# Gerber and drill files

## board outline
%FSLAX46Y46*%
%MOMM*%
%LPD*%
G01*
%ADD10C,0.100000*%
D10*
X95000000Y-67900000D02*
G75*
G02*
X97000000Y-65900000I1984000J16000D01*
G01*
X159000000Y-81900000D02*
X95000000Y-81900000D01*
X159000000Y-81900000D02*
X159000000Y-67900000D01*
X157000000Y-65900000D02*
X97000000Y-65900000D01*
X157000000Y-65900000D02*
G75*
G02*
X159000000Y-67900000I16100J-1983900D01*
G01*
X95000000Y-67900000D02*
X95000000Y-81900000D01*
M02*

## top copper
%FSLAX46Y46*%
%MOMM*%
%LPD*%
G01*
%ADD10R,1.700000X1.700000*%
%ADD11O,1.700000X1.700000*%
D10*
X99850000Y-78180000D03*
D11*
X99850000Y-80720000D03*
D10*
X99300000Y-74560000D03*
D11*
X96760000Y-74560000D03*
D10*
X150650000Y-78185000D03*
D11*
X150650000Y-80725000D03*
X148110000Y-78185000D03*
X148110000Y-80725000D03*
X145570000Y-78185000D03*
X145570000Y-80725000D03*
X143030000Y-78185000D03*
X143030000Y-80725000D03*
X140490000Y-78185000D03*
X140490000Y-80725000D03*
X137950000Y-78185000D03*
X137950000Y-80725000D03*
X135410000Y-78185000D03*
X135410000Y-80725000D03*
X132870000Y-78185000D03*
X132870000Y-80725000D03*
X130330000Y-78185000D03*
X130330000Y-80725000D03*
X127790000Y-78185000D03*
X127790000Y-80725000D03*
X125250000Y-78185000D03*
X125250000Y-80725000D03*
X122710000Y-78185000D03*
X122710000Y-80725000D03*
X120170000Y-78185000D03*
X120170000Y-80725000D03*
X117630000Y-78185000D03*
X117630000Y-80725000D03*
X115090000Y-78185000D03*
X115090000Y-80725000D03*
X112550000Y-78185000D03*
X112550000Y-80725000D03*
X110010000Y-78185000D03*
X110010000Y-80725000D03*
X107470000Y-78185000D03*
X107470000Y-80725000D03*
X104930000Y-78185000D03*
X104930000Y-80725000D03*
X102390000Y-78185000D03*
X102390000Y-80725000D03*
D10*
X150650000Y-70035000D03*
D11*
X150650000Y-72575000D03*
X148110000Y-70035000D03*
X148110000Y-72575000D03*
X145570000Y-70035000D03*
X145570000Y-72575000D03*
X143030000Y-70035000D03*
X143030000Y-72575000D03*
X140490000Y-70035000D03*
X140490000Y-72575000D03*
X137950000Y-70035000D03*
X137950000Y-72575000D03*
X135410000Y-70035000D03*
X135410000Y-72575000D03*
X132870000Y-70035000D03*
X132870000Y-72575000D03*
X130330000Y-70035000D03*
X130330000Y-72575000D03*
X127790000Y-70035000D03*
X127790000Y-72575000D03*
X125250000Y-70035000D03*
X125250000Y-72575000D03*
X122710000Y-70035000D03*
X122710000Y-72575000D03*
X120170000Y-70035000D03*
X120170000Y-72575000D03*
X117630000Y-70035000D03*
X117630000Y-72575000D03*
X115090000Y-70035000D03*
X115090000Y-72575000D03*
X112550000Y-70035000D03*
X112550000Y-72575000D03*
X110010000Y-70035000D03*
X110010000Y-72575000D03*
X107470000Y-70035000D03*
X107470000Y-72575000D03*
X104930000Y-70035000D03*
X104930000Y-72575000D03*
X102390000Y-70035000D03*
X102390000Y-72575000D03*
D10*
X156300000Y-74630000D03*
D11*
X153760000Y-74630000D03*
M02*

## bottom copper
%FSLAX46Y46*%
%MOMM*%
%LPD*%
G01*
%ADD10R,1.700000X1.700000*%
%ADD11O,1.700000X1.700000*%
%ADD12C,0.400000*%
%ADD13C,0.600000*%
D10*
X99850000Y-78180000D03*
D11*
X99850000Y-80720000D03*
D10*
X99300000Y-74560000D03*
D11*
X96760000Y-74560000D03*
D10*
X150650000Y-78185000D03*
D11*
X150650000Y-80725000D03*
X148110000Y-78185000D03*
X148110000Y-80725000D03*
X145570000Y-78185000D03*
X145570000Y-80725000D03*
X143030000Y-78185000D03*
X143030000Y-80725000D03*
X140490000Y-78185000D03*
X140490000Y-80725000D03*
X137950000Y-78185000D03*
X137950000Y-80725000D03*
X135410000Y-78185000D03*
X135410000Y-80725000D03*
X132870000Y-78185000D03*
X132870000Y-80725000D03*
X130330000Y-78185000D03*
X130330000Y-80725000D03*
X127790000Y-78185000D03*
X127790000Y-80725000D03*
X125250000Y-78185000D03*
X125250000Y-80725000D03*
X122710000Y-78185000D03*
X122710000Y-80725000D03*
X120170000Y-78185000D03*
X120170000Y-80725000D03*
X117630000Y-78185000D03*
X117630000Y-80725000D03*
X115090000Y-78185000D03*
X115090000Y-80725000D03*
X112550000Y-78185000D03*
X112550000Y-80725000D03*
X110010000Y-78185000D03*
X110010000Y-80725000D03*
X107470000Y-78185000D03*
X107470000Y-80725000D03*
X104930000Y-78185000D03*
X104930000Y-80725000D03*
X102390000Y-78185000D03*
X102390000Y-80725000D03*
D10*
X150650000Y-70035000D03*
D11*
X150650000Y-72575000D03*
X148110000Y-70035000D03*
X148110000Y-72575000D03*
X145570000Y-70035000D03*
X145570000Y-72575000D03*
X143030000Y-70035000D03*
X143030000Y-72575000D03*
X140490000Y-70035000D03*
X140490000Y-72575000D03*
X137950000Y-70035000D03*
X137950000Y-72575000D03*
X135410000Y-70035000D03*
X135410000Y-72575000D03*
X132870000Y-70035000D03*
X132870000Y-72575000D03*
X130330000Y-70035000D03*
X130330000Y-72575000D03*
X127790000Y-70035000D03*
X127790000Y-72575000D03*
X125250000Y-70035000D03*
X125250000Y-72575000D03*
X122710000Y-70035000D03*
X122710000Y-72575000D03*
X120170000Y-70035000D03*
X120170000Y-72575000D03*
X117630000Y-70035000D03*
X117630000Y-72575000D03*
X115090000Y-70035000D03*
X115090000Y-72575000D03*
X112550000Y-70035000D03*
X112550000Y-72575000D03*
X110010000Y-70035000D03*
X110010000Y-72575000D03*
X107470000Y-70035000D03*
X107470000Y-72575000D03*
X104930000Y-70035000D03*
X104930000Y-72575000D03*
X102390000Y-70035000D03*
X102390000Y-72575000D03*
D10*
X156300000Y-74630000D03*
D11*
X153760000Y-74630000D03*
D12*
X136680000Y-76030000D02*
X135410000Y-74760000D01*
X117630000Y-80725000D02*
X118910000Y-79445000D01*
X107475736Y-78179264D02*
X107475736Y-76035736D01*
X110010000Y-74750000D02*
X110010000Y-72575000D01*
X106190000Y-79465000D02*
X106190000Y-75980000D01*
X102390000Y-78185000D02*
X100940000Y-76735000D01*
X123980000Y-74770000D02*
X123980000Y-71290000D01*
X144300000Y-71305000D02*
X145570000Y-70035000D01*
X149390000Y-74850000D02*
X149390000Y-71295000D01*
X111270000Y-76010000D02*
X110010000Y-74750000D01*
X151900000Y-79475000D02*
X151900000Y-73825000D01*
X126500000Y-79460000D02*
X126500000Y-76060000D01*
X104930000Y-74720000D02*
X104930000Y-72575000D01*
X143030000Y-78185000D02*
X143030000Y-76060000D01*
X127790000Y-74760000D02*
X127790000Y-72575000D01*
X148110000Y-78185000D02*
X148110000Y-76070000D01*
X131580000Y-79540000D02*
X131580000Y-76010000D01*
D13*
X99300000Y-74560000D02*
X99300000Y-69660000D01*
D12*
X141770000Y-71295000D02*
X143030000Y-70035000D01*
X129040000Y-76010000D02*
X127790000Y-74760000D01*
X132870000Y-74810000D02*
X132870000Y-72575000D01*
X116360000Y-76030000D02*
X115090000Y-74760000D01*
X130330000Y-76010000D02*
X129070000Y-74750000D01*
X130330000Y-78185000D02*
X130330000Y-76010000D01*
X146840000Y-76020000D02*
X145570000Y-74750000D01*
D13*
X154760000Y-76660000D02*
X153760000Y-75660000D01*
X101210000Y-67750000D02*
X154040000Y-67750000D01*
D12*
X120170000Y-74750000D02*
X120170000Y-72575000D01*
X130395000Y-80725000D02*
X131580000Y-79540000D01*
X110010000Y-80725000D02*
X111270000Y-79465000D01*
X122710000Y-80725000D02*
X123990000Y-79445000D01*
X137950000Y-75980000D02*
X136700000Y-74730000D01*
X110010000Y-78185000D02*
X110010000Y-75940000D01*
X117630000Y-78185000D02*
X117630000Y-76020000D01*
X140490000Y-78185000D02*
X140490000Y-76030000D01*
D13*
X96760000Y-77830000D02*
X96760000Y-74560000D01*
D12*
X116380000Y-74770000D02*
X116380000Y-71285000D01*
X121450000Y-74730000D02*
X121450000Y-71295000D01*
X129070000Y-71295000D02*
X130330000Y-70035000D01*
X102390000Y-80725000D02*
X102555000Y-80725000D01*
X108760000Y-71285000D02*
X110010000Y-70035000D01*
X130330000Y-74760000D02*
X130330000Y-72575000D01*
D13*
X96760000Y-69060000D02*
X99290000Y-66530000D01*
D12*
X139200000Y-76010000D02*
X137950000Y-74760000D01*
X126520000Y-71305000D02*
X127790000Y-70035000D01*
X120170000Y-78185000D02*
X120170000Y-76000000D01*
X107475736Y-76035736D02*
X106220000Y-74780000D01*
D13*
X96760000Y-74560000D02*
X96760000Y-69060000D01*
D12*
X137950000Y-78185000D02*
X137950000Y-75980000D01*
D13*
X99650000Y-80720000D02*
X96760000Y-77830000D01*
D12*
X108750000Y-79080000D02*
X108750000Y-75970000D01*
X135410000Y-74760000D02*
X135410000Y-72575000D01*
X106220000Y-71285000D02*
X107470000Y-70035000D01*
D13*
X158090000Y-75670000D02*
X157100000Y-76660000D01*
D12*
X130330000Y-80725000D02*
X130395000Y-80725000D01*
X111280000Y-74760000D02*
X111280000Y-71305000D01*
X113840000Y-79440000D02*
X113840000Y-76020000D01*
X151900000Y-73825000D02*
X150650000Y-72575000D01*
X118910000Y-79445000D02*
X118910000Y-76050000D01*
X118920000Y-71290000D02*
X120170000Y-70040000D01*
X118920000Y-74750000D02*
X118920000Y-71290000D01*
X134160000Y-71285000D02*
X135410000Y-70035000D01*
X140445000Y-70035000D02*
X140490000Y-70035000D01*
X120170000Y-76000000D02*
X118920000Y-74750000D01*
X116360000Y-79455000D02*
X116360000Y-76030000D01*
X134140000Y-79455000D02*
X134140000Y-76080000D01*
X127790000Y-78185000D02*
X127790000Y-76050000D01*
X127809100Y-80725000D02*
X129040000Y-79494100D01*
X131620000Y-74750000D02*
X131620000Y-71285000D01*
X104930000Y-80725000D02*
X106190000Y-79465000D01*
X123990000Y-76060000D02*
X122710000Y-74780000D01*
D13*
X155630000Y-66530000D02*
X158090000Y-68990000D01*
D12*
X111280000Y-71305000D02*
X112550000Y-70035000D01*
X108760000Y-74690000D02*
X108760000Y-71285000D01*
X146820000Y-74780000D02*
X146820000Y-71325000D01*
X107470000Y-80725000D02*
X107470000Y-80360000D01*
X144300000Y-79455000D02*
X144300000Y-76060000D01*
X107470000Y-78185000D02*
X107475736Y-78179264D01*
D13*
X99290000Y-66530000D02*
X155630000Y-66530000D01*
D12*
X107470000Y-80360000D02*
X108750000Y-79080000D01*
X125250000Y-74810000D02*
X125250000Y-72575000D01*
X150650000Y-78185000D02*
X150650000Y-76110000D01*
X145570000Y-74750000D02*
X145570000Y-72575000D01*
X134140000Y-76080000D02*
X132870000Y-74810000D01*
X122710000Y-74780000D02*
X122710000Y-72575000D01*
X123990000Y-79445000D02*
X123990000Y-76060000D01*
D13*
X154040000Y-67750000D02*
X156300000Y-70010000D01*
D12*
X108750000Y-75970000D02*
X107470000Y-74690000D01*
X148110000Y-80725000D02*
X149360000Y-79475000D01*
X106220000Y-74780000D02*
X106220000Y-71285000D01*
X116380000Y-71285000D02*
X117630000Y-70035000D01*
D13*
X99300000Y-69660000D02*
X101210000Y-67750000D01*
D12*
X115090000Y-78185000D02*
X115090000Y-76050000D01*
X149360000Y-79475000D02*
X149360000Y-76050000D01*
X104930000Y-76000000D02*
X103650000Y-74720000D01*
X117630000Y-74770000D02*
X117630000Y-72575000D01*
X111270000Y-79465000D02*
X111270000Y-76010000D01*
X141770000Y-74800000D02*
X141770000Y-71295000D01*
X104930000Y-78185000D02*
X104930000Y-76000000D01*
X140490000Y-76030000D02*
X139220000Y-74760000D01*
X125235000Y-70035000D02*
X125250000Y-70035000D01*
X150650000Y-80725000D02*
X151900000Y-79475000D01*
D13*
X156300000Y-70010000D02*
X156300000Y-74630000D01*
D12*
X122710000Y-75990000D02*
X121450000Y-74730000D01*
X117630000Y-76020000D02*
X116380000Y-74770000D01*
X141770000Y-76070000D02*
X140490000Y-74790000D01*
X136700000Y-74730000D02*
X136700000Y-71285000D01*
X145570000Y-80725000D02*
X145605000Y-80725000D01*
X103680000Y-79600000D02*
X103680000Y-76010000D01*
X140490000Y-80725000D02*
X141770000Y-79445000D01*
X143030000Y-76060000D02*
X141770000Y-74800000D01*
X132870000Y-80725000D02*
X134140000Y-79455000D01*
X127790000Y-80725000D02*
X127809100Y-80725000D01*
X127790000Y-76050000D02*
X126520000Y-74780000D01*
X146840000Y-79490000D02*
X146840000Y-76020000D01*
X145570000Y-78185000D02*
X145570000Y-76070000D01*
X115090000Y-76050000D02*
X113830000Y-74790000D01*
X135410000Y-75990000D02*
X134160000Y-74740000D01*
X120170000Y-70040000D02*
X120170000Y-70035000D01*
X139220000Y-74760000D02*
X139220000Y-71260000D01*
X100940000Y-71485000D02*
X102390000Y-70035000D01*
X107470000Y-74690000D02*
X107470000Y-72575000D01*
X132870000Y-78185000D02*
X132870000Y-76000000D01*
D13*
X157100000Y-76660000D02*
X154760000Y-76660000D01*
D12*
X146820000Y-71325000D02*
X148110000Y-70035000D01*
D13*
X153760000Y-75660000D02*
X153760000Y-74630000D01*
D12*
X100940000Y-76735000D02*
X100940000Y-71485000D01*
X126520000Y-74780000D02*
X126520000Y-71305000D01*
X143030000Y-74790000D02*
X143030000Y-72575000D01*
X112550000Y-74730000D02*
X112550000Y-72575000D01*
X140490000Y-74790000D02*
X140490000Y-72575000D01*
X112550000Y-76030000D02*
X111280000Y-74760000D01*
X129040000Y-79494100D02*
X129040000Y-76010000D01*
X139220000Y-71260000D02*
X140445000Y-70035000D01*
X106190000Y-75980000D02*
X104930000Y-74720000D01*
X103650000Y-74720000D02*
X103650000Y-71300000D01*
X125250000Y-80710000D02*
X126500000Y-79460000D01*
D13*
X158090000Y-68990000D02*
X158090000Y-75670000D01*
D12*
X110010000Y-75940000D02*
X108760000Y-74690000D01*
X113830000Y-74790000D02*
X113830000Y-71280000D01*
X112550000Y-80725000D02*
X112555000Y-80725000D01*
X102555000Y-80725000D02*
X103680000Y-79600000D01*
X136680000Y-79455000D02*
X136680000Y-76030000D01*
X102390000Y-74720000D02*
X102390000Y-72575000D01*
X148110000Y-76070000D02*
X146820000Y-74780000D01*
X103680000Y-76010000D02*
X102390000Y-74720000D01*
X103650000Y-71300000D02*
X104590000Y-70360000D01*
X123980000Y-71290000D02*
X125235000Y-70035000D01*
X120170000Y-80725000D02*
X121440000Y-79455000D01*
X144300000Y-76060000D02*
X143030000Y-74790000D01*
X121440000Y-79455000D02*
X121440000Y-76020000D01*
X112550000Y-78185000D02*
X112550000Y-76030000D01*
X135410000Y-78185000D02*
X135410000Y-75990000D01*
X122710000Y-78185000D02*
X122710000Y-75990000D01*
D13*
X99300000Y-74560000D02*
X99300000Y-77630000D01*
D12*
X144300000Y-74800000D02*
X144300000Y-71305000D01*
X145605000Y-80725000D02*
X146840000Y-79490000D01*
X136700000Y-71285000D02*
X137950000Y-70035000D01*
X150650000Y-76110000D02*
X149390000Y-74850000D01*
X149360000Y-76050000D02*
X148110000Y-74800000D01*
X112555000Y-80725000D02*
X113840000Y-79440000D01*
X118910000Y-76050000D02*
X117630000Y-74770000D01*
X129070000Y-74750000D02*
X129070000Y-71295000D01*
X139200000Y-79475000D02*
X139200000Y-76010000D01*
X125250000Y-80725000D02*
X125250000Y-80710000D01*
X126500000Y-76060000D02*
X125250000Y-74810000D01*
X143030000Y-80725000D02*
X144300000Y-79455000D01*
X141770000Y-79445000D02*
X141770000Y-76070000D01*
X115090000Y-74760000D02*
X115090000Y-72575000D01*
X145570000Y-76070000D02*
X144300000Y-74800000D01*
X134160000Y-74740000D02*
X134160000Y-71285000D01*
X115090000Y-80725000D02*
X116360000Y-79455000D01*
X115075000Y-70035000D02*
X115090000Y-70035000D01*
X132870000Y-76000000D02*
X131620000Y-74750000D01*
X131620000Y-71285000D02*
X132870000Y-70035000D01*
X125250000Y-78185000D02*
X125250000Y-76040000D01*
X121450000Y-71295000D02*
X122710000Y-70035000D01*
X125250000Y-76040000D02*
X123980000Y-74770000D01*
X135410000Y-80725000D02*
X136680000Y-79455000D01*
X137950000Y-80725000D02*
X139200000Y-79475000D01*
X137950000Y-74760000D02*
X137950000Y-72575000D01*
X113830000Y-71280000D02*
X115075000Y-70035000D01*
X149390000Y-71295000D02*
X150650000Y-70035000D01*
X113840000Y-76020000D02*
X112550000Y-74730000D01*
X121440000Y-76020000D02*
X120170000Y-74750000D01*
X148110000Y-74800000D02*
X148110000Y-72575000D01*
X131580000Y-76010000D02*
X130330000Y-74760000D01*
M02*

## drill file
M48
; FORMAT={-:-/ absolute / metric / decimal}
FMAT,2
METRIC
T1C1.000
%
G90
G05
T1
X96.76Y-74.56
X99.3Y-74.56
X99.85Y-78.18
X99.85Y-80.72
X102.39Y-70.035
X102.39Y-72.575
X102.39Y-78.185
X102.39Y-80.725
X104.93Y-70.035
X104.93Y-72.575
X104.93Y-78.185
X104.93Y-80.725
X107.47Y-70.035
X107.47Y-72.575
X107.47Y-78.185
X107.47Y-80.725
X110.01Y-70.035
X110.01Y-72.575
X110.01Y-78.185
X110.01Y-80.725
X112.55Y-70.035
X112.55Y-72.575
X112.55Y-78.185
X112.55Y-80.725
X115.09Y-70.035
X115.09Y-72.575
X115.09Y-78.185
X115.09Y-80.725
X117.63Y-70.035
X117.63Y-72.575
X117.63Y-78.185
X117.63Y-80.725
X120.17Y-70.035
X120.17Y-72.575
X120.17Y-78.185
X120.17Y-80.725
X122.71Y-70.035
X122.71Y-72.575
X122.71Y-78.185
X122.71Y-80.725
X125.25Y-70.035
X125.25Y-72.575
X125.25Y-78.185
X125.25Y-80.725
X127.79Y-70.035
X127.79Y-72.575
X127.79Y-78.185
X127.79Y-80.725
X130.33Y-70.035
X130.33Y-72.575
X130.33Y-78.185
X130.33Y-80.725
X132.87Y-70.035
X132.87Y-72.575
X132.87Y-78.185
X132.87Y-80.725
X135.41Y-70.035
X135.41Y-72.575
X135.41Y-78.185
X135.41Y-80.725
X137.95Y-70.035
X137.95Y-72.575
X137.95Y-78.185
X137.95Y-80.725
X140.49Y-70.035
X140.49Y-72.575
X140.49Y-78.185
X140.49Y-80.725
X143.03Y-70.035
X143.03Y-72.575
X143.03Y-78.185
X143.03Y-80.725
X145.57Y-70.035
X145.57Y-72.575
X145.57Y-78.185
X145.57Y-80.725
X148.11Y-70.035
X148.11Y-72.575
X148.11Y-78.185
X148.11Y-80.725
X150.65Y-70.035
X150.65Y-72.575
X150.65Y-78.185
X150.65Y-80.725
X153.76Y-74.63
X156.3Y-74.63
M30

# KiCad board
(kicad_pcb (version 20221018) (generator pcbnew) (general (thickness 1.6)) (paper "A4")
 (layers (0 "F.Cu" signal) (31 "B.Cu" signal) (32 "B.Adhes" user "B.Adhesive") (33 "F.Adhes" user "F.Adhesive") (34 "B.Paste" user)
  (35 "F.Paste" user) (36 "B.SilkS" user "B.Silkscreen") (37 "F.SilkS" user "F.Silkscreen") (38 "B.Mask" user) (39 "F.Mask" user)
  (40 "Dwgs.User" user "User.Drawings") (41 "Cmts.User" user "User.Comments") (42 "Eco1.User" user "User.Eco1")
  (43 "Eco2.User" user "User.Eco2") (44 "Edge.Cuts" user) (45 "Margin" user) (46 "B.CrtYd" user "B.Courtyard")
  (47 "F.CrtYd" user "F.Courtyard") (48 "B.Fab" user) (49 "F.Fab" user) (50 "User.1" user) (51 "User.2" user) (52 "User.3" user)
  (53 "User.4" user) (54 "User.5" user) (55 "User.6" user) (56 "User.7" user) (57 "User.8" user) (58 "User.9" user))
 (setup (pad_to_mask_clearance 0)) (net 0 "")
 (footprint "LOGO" (layer "F.Cu") (at 126.5 75.56)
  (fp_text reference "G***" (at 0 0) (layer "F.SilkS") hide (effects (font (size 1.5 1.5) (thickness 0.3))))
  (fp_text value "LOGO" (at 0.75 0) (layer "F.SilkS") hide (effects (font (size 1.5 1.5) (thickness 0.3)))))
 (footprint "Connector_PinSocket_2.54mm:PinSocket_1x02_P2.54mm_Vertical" (layer "B.Cu") (at 99.85 78.18 180)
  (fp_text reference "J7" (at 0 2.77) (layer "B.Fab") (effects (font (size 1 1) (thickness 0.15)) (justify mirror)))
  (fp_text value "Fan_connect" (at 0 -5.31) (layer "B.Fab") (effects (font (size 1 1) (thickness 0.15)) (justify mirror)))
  (pad "1" thru_hole rect (at 0 0 180) (size 1.7 1.7) (drill 1) (layers "*.Cu" "*.Mask"))
  (pad "2" thru_hole oval (at 0 -2.54 180) (size 1.7 1.7) (drill 1) (layers "*.Cu" "*.Mask")))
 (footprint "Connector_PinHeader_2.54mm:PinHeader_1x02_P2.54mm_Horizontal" (layer "B.Cu") (at 99.3 74.56 90)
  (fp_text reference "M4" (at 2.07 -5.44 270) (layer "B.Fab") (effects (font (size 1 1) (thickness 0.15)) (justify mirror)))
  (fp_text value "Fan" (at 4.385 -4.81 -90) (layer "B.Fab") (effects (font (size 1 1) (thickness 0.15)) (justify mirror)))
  (pad "1" thru_hole rect (at 0 0 90) (size 1.7 1.7) (drill 1) (layers "*.Cu" "*.Mask"))
  (pad "2" thru_hole oval (at 0 -2.54 90) (size 1.7 1.7) (drill 1) (layers "*.Cu" "*.Mask")))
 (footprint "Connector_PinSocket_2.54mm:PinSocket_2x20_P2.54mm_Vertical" (layer "B.Cu") (at 126.49 79.455 90)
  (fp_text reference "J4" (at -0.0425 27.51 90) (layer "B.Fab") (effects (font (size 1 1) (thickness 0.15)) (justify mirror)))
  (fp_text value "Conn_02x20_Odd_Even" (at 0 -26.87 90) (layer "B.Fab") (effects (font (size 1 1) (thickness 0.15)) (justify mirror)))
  (pad "1" thru_hole rect (at 1.27 24.16 90) (size 1.7 1.7) (drill 1) (layers "*.Cu" "*.Mask"))
  (pad "2" thru_hole oval (at -1.27 24.16 90) (size 1.7 1.7) (drill 1) (layers "*.Cu" "*.Mask"))
  (pad "3" thru_hole oval (at 1.27 21.62 90) (size 1.7 1.7) (drill 1) (layers "*.Cu" "*.Mask"))
  (pad "4" thru_hole oval (at -1.27 21.62 90) (size 1.7 1.7) (drill 1) (layers "*.Cu" "*.Mask"))
  (pad "5" thru_hole oval (at 1.27 19.08 90) (size 1.7 1.7) (drill 1) (layers "*.Cu" "*.Mask"))
  (pad "6" thru_hole oval (at -1.27 19.08 90) (size 1.7 1.7) (drill 1) (layers "*.Cu" "*.Mask"))
  (pad "7" thru_hole oval (at 1.27 16.54 90) (size 1.7 1.7) (drill 1) (layers "*.Cu" "*.Mask"))
  (pad "8" thru_hole oval (at -1.27 16.54 90) (size 1.7 1.7) (drill 1) (layers "*.Cu" "*.Mask"))
  (pad "9" thru_hole oval (at 1.27 14 90) (size 1.7 1.7) (drill 1) (layers "*.Cu" "*.Mask"))
  (pad "10" thru_hole oval (at -1.27 14 90) (size 1.7 1.7) (drill 1) (layers "*.Cu" "*.Mask"))
  (pad "11" thru_hole oval (at 1.27 11.46 90) (size 1.7 1.7) (drill 1) (layers "*.Cu" "*.Mask"))
  (pad "12" thru_hole oval (at -1.27 11.46 90) (size 1.7 1.7) (drill 1) (layers "*.Cu" "*.Mask"))
  (pad "13" thru_hole oval (at 1.27 8.92 90) (size 1.7 1.7) (drill 1) (layers "*.Cu" "*.Mask"))
  (pad "14" thru_hole oval (at -1.27 8.92 90) (size 1.7 1.7) (drill 1) (layers "*.Cu" "*.Mask"))
  (pad "15" thru_hole oval (at 1.27 6.38 90) (size 1.7 1.7) (drill 1) (layers "*.Cu" "*.Mask"))
  (pad "16" thru_hole oval (at -1.27 6.38 90) (size 1.7 1.7) (drill 1) (layers "*.Cu" "*.Mask"))
  (pad "17" thru_hole oval (at 1.27 3.84 90) (size 1.7 1.7) (drill 1) (layers "*.Cu" "*.Mask"))
  (pad "18" thru_hole oval (at -1.27 3.84 90) (size 1.7 1.7) (drill 1) (layers "*.Cu" "*.Mask"))
  (pad "19" thru_hole oval (at 1.27 1.3 90) (size 1.7 1.7) (drill 1) (layers "*.Cu" "*.Mask"))
  (pad "20" thru_hole oval (at -1.27 1.3 90) (size 1.7 1.7) (drill 1) (layers "*.Cu" "*.Mask"))
  (pad "21" thru_hole oval (at 1.27 -1.24 90) (size 1.7 1.7) (drill 1) (layers "*.Cu" "*.Mask"))
  (pad "22" thru_hole oval (at -1.27 -1.24 90) (size 1.7 1.7) (drill 1) (layers "*.Cu" "*.Mask"))
  (pad "23" thru_hole oval (at 1.27 -3.78 90) (size 1.7 1.7) (drill 1) (layers "*.Cu" "*.Mask"))
  (pad "24" thru_hole oval (at -1.27 -3.78 90) (size 1.7 1.7) (drill 1) (layers "*.Cu" "*.Mask"))
  (pad "25" thru_hole oval (at 1.27 -6.32 90) (size 1.7 1.7) (drill 1) (layers "*.Cu" "*.Mask"))
  (pad "26" thru_hole oval (at -1.27 -6.32 90) (size 1.7 1.7) (drill 1) (layers "*.Cu" "*.Mask"))
  (pad "27" thru_hole oval (at 1.27 -8.86 90) (size 1.7 1.7) (drill 1) (layers "*.Cu" "*.Mask"))
  (pad "28" thru_hole oval (at -1.27 -8.86 90) (size 1.7 1.7) (drill 1) (layers "*.Cu" "*.Mask"))
  (pad "29" thru_hole oval (at 1.27 -11.4 90) (size 1.7 1.7) (drill 1) (layers "*.Cu" "*.Mask"))
  (pad "30" thru_hole oval (at -1.27 -11.4 90) (size 1.7 1.7) (drill 1) (layers "*.Cu" "*.Mask"))
  (pad "31" thru_hole oval (at 1.27 -13.94 90) (size 1.7 1.7) (drill 1) (layers "*.Cu" "*.Mask"))
  (pad "32" thru_hole oval (at -1.27 -13.94 90) (size 1.7 1.7) (drill 1) (layers "*.Cu" "*.Mask"))
  (pad "33" thru_hole oval (at 1.27 -16.48 90) (size 1.7 1.7) (drill 1) (layers "*.Cu" "*.Mask"))
  (pad "34" thru_hole oval (at -1.27 -16.48 90) (size 1.7 1.7) (drill 1) (layers "*.Cu" "*.Mask"))
  (pad "35" thru_hole oval (at 1.27 -19.02 90) (size 1.7 1.7) (drill 1) (layers "*.Cu" "*.Mask"))
  (pad "36" thru_hole oval (at -1.27 -19.02 90) (size 1.7 1.7) (drill 1) (layers "*.Cu" "*.Mask"))
  (pad "37" thru_hole oval (at 1.27 -21.56 90) (size 1.7 1.7) (drill 1) (layers "*.Cu" "*.Mask"))
  (pad "38" thru_hole oval (at -1.27 -21.56 90) (size 1.7 1.7) (drill 1) (layers "*.Cu" "*.Mask"))
  (pad "39" thru_hole oval (at 1.27 -24.1 90) (size 1.7 1.7) (drill 1) (layers "*.Cu" "*.Mask"))
  (pad "40" thru_hole oval (at -1.27 -24.1 90) (size 1.7 1.7) (drill 1) (layers "*.Cu" "*.Mask")))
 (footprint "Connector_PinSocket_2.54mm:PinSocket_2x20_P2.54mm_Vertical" (layer "B.Cu") (at 126.49 71.305 90)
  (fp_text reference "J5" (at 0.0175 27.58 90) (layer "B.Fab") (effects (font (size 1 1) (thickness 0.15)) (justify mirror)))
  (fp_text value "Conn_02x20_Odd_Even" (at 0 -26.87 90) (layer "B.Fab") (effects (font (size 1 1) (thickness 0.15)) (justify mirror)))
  (pad "1" thru_hole rect (at 1.27 24.16 90) (size 1.7 1.7) (drill 1) (layers "*.Cu" "*.Mask"))
  (pad "2" thru_hole oval (at -1.27 24.16 90) (size 1.7 1.7) (drill 1) (layers "*.Cu" "*.Mask"))
  (pad "3" thru_hole oval (at 1.27 21.62 90) (size 1.7 1.7) (drill 1) (layers "*.Cu" "*.Mask"))
  (pad "4" thru_hole oval (at -1.27 21.62 90) (size 1.7 1.7) (drill 1) (layers "*.Cu" "*.Mask"))
  (pad "5" thru_hole oval (at 1.27 19.08 90) (size 1.7 1.7) (drill 1) (layers "*.Cu" "*.Mask"))
  (pad "6" thru_hole oval (at -1.27 19.08 90) (size 1.7 1.7) (drill 1) (layers "*.Cu" "*.Mask"))
  (pad "7" thru_hole oval (at 1.27 16.54 90) (size 1.7 1.7) (drill 1) (layers "*.Cu" "*.Mask"))
  (pad "8" thru_hole oval (at -1.27 16.54 90) (size 1.7 1.7) (drill 1) (layers "*.Cu" "*.Mask"))
  (pad "9" thru_hole oval (at 1.27 14 90) (size 1.7 1.7) (drill 1) (layers "*.Cu" "*.Mask"))
  (pad "10" thru_hole oval (at -1.27 14 90) (size 1.7 1.7) (drill 1) (layers "*.Cu" "*.Mask"))
  (pad "11" thru_hole oval (at 1.27 11.46 90) (size 1.7 1.7) (drill 1) (layers "*.Cu" "*.Mask"))
  (pad "12" thru_hole oval (at -1.27 11.46 90) (size 1.7 1.7) (drill 1) (layers "*.Cu" "*.Mask"))
  (pad "13" thru_hole oval (at 1.27 8.92 90) (size 1.7 1.7) (drill 1) (layers "*.Cu" "*.Mask"))
  (pad "14" thru_hole oval (at -1.27 8.92 90) (size 1.7 1.7) (drill 1) (layers "*.Cu" "*.Mask"))
  (pad "15" thru_hole oval (at 1.27 6.38 90) (size 1.7 1.7) (drill 1) (layers "*.Cu" "*.Mask"))
  (pad "16" thru_hole oval (at -1.27 6.38 90) (size 1.7 1.7) (drill 1) (layers "*.Cu" "*.Mask"))
  (pad "17" thru_hole oval (at 1.27 3.84 90) (size 1.7 1.7) (drill 1) (layers "*.Cu" "*.Mask"))
  (pad "18" thru_hole oval (at -1.27 3.84 90) (size 1.7 1.7) (drill 1) (layers "*.Cu" "*.Mask"))
  (pad "19" thru_hole oval (at 1.27 1.3 90) (size 1.7 1.7) (drill 1) (layers "*.Cu" "*.Mask"))
  (pad "20" thru_hole oval (at -1.27 1.3 90) (size 1.7 1.7) (drill 1) (layers "*.Cu" "*.Mask"))
  (pad "21" thru_hole oval (at 1.27 -1.24 90) (size 1.7 1.7) (drill 1) (layers "*.Cu" "*.Mask"))
  (pad "22" thru_hole oval (at -1.27 -1.24 90) (size 1.7 1.7) (drill 1) (layers "*.Cu" "*.Mask"))
  (pad "23" thru_hole oval (at 1.27 -3.78 90) (size 1.7 1.7) (drill 1) (layers "*.Cu" "*.Mask"))
  (pad "24" thru_hole oval (at -1.27 -3.78 90) (size 1.7 1.7) (drill 1) (layers "*.Cu" "*.Mask"))
  (pad "25" thru_hole oval (at 1.27 -6.32 90) (size 1.7 1.7) (drill 1) (layers "*.Cu" "*.Mask"))
  (pad "26" thru_hole oval (at -1.27 -6.32 90) (size 1.7 1.7) (drill 1) (layers "*.Cu" "*.Mask"))
  (pad "27" thru_hole oval (at 1.27 -8.86 90) (size 1.7 1.7) (drill 1) (layers "*.Cu" "*.Mask"))
  (pad "28" thru_hole oval (at -1.27 -8.86 90) (size 1.7 1.7) (drill 1) (layers "*.Cu" "*.Mask"))
  (pad "29" thru_hole oval (at 1.27 -11.4 90) (size 1.7 1.7) (drill 1) (layers "*.Cu" "*.Mask"))
  (pad "30" thru_hole oval (at -1.27 -11.4 90) (size 1.7 1.7) (drill 1) (layers "*.Cu" "*.Mask"))
  (pad "31" thru_hole oval (at 1.27 -13.94 90) (size 1.7 1.7) (drill 1) (layers "*.Cu" "*.Mask"))
  (pad "32" thru_hole oval (at -1.27 -13.94 90) (size 1.7 1.7) (drill 1) (layers "*.Cu" "*.Mask"))
  (pad "33" thru_hole oval (at 1.27 -16.48 90) (size 1.7 1.7) (drill 1) (layers "*.Cu" "*.Mask"))
  (pad "34" thru_hole oval (at -1.27 -16.48 90) (size 1.7 1.7) (drill 1) (layers "*.Cu" "*.Mask"))
  (pad "35" thru_hole oval (at 1.27 -19.02 90) (size 1.7 1.7) (drill 1) (layers "*.Cu" "*.Mask"))
  (pad "36" thru_hole oval (at -1.27 -19.02 90) (size 1.7 1.7) (drill 1) (layers "*.Cu" "*.Mask"))
  (pad "37" thru_hole oval (at 1.27 -21.56 90) (size 1.7 1.7) (drill 1) (layers "*.Cu" "*.Mask"))
  (pad "38" thru_hole oval (at -1.27 -21.56 90) (size 1.7 1.7) (drill 1) (layers "*.Cu" "*.Mask"))
  (pad "39" thru_hole oval (at 1.27 -24.1 90) (size 1.7 1.7) (drill 1) (layers "*.Cu" "*.Mask"))
  (pad "40" thru_hole oval (at -1.27 -24.1 90) (size 1.7 1.7) (drill 1) (layers "*.Cu" "*.Mask")))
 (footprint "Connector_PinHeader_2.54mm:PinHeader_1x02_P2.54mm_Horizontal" (layer "B.Cu") (at 156.3 74.63 90)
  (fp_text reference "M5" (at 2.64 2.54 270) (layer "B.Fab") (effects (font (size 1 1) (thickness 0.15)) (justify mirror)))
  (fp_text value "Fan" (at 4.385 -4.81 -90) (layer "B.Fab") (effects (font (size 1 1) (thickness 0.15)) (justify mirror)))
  (pad "1" thru_hole rect (at 0 0 90) (size 1.7 1.7) (drill 1) (layers "*.Cu" "*.Mask"))
  (pad "2" thru_hole oval (at 0 -2.54 90) (size 1.7 1.7) (drill 1) (layers "*.Cu" "*.Mask")))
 (gr_arc (start 95 67.9) (mid 95.581055 66.481055) (end 97 65.9) (stroke (width 0.1) (type default)) (layer "Edge.Cuts"))
 (gr_line (start 159 81.9) (end 95 81.9) (stroke (width 0.1) (type default)) (layer "Edge.Cuts"))
 (gr_line (start 159 81.9) (end 159 67.9) (stroke (width 0.1) (type default)) (layer "Edge.Cuts"))
 (gr_line (start 157 65.9) (end 97 65.9) (stroke (width 0.1) (type default)) (layer "Edge.Cuts"))
 (gr_arc (start 157 65.9) (mid 158.418975 66.481025) (end 159 67.9) (stroke (width 0.1) (type default)) (layer "Edge.Cuts"))
 (gr_line (start 95 67.9) (end 95 81.9) (stroke (width 0.1) (type default)) (layer "Edge.Cuts"))
 (segment (start 136.68 76.03) (end 135.41 74.76) (width 0.4) (layer "B.Cu") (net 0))
 (segment (start 117.63 80.725) (end 118.91 79.445) (width 0.4) (layer "B.Cu") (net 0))
 (segment (start 107.475736 78.179264) (end 107.475736 76.035736) (width 0.4) (layer "B.Cu") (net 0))
 (segment (start 110.01 74.75) (end 110.01 72.575) (width 0.4) (layer "B.Cu") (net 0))
 (segment (start 106.19 79.465) (end 106.19 75.98) (width 0.4) (layer "B.Cu") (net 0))
 (segment (start 102.39 78.185) (end 100.94 76.735) (width 0.4) (layer "B.Cu") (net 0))
 (segment (start 123.98 74.77) (end 123.98 71.29) (width 0.4) (layer "B.Cu") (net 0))
 (segment (start 144.3 71.305) (end 145.57 70.035) (width 0.4) (layer "B.Cu") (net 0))
 (segment (start 149.39 74.85) (end 149.39 71.295) (width 0.4) (layer "B.Cu") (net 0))
 (segment (start 111.27 76.01) (end 110.01 74.75) (width 0.4) (layer "B.Cu") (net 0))
 (segment (start 151.9 79.475) (end 151.9 73.825) (width 0.4) (layer "B.Cu") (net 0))
 (segment (start 126.5 79.46) (end 126.5 76.06) (width 0.4) (layer "B.Cu") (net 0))
 (segment (start 104.93 74.72) (end 104.93 72.575) (width 0.4) (layer "B.Cu") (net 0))
 (segment (start 143.03 78.185) (end 143.03 76.06) (width 0.4) (layer "B.Cu") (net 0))
 (segment (start 127.79 74.76) (end 127.79 72.575) (width 0.4) (layer "B.Cu") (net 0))
 (segment (start 148.11 78.185) (end 148.11 76.07) (width 0.4) (layer "B.Cu") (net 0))
 (segment (start 131.58 79.54) (end 131.58 76.01) (width 0.4) (layer "B.Cu") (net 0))
 (segment (start 99.3 74.56) (end 99.3 69.66) (width 0.6) (layer "B.Cu") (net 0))
 (segment (start 141.77 71.295) (end 143.03 70.035) (width 0.4) (layer "B.Cu") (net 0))
 (segment (start 129.04 76.01) (end 127.79 74.76) (width 0.4) (layer "B.Cu") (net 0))
 (segment (start 132.87 74.81) (end 132.87 72.575) (width 0.4) (layer "B.Cu") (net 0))
 (segment (start 116.36 76.03) (end 115.09 74.76) (width 0.4) (layer "B.Cu") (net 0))
 (segment (start 130.33 76.01) (end 129.07 74.75) (width 0.4) (layer "B.Cu") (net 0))
 (segment (start 130.33 78.185) (end 130.33 76.01) (width 0.4) (layer "B.Cu") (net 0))
 (segment (start 146.84 76.02) (end 145.57 74.75) (width 0.4) (layer "B.Cu") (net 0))
 (segment (start 154.76 76.66) (end 153.76 75.66) (width 0.6) (layer "B.Cu") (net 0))
 (segment (start 101.21 67.75) (end 154.04 67.75) (width 0.6) (layer "B.Cu") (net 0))
 (segment (start 120.17 74.75) (end 120.17 72.575) (width 0.4) (layer "B.Cu") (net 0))
 (segment (start 130.395 80.725) (end 131.58 79.54) (width 0.4) (layer "B.Cu") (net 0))
 (segment (start 110.01 80.725) (end 111.27 79.465) (width 0.4) (layer "B.Cu") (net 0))
 (segment (start 122.71 80.725) (end 123.99 79.445) (width 0.4) (layer "B.Cu") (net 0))
 (segment (start 137.95 75.98) (end 136.7 74.73) (width 0.4) (layer "B.Cu") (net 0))
 (segment (start 110.01 78.185) (end 110.01 75.94) (width 0.4) (layer "B.Cu") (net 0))
 (segment (start 117.63 78.185) (end 117.63 76.02) (width 0.4) (layer "B.Cu") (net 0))
 (segment (start 140.49 78.185) (end 140.49 76.03) (width 0.4) (layer "B.Cu") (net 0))
 (segment (start 96.76 77.83) (end 96.76 74.56) (width 0.6) (layer "B.Cu") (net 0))
 (segment (start 116.38 74.77) (end 116.38 71.285) (width 0.4) (layer "B.Cu") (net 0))
 (segment (start 121.45 74.73) (end 121.45 71.295) (width 0.4) (layer "B.Cu") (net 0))
 (segment (start 129.07 71.295) (end 130.33 70.035) (width 0.4) (layer "B.Cu") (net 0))
 (segment (start 102.39 80.725) (end 102.555 80.725) (width 0.4) (layer "B.Cu") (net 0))
 (segment (start 108.76 71.285) (end 110.01 70.035) (width 0.4) (layer "B.Cu") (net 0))
 (segment (start 130.33 74.76) (end 130.33 72.575) (width 0.4) (layer "B.Cu") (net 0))
 (segment (start 96.76 69.06) (end 99.29 66.53) (width 0.6) (layer "B.Cu") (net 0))
 (segment (start 139.2 76.01) (end 137.95 74.76) (width 0.4) (layer "B.Cu") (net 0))
 (segment (start 126.52 71.305) (end 127.79 70.035) (width 0.4) (layer "B.Cu") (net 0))
 (segment (start 120.17 78.185) (end 120.17 76) (width 0.4) (layer "B.Cu") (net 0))
 (segment (start 107.475736 76.035736) (end 106.22 74.78) (width 0.4) (layer "B.Cu") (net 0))
 (segment (start 96.76 74.56) (end 96.76 69.06) (width 0.6) (layer "B.Cu") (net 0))
 (segment (start 137.95 78.185) (end 137.95 75.98) (width 0.4) (layer "B.Cu") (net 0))
 (segment (start 99.65 80.72) (end 96.76 77.83) (width 0.6) (layer "B.Cu") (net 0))
 (segment (start 108.75 79.08) (end 108.75 75.97) (width 0.4) (layer "B.Cu") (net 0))
 (segment (start 135.41 74.76) (end 135.41 72.575) (width 0.4) (layer "B.Cu") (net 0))
 (segment (start 106.22 71.285) (end 107.47 70.035) (width 0.4) (layer "B.Cu") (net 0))
 (segment (start 158.09 75.67) (end 157.1 76.66) (width 0.6) (layer "B.Cu") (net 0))
 (segment (start 130.33 80.725) (end 130.395 80.725) (width 0.4) (layer "B.Cu") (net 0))
 (segment (start 111.28 74.76) (end 111.28 71.305) (width 0.4) (layer "B.Cu") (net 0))
 (segment (start 113.84 79.44) (end 113.84 76.02) (width 0.4) (layer "B.Cu") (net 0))
 (segment (start 151.9 73.825) (end 150.65 72.575) (width 0.4) (layer "B.Cu") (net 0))
 (segment (start 118.91 79.445) (end 118.91 76.05) (width 0.4) (layer "B.Cu") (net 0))
 (segment (start 118.92 71.29) (end 120.17 70.04) (width 0.4) (layer "B.Cu") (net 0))
 (segment (start 118.92 74.75) (end 118.92 71.29) (width 0.4) (layer "B.Cu") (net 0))
 (segment (start 134.16 71.285) (end 135.41 70.035) (width 0.4) (layer "B.Cu") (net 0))
 (segment (start 140.445 70.035) (end 140.49 70.035) (width 0.4) (layer "B.Cu") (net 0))
 (segment (start 120.17 76) (end 118.92 74.75) (width 0.4) (layer "B.Cu") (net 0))
 (segment (start 116.36 79.455) (end 116.36 76.03) (width 0.4) (layer "B.Cu") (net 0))
 (segment (start 134.14 79.455) (end 134.14 76.08) (width 0.4) (layer "B.Cu") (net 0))
 (segment (start 127.79 78.185) (end 127.79 76.05) (width 0.4) (layer "B.Cu") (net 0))
 (segment (start 127.8091 80.725) (end 129.04 79.4941) (width 0.4) (layer "B.Cu") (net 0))
 (segment (start 131.62 74.75) (end 131.62 71.285) (width 0.4) (layer "B.Cu") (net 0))
 (segment (start 104.93 80.725) (end 106.19 79.465) (width 0.4) (layer "B.Cu") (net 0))
 (segment (start 123.99 76.06) (end 122.71 74.78) (width 0.4) (layer "B.Cu") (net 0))
 (segment (start 155.63 66.53) (end 158.09 68.99) (width 0.6) (layer "B.Cu") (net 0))
 (segment (start 111.28 71.305) (end 112.55 70.035) (width 0.4) (layer "B.Cu") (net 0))
 (segment (start 108.76 74.69) (end 108.76 71.285) (width 0.4) (layer "B.Cu") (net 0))
 (segment (start 146.82 74.78) (end 146.82 71.325) (width 0.4) (layer "B.Cu") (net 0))
 (segment (start 107.47 80.725) (end 107.47 80.36) (width 0.4) (layer "B.Cu") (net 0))
 (segment (start 144.3 79.455) (end 144.3 76.06) (width 0.4) (layer "B.Cu") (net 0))
 (segment (start 107.47 78.185) (end 107.475736 78.179264) (width 0.4) (layer "B.Cu") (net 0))
 (segment (start 99.29 66.53) (end 155.63 66.53) (width 0.6) (layer "B.Cu") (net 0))
 (segment (start 107.47 80.36) (end 108.75 79.08) (width 0.4) (layer "B.Cu") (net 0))
 (segment (start 125.25 74.81) (end 125.25 72.575) (width 0.4) (layer "B.Cu") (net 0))
 (segment (start 150.65 78.185) (end 150.65 76.11) (width 0.4) (layer "B.Cu") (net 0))
 (segment (start 145.57 74.75) (end 145.57 72.575) (width 0.4) (layer "B.Cu") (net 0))
 (segment (start 134.14 76.08) (end 132.87 74.81) (width 0.4) (layer "B.Cu") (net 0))
 (segment (start 122.71 74.78) (end 122.71 72.575) (width 0.4) (layer "B.Cu") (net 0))
 (segment (start 123.99 79.445) (end 123.99 76.06) (width 0.4) (layer "B.Cu") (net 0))
 (segment (start 154.04 67.75) (end 156.3 70.01) (width 0.6) (layer "B.Cu") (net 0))
 (segment (start 108.75 75.97) (end 107.47 74.69) (width 0.4) (layer "B.Cu") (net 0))
 (segment (start 148.11 80.725) (end 149.36 79.475) (width 0.4) (layer "B.Cu") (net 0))
 (segment (start 106.22 74.78) (end 106.22 71.285) (width 0.4) (layer "B.Cu") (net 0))
 (segment (start 116.38 71.285) (end 117.63 70.035) (width 0.4) (layer "B.Cu") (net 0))
 (segment (start 99.3 69.66) (end 101.21 67.75) (width 0.6) (layer "B.Cu") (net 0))
 (segment (start 115.09 78.185) (end 115.09 76.05) (width 0.4) (layer "B.Cu") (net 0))
 (segment (start 149.36 79.475) (end 149.36 76.05) (width 0.4) (layer "B.Cu") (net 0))
 (segment (start 104.93 76) (end 103.65 74.72) (width 0.4) (layer "B.Cu") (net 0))
 (segment (start 117.63 74.77) (end 117.63 72.575) (width 0.4) (layer "B.Cu") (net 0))
 (segment (start 111.27 79.465) (end 111.27 76.01) (width 0.4) (layer "B.Cu") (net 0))
 (segment (start 141.77 74.8) (end 141.77 71.295) (width 0.4) (layer "B.Cu") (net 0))
 (segment (start 104.93 78.185) (end 104.93 76) (width 0.4) (layer "B.Cu") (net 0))
 (segment (start 140.49 76.03) (end 139.22 74.76) (width 0.4) (layer "B.Cu") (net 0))
 (segment (start 125.235 70.035) (end 125.25 70.035) (width 0.4) (layer "B.Cu") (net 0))
 (segment (start 150.65 80.725) (end 151.9 79.475) (width 0.4) (layer "B.Cu") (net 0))
 (segment (start 156.3 70.01) (end 156.3 74.63) (width 0.6) (layer "B.Cu") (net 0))
 (segment (start 122.71 75.99) (end 121.45 74.73) (width 0.4) (layer "B.Cu") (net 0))
 (segment (start 117.63 76.02) (end 116.38 74.77) (width 0.4) (layer "B.Cu") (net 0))
 (segment (start 141.77 76.07) (end 140.49 74.79) (width 0.4) (layer "B.Cu") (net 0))
 (segment (start 136.7 74.73) (end 136.7 71.285) (width 0.4) (layer "B.Cu") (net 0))
 (segment (start 145.57 80.725) (end 145.605 80.725) (width 0.4) (layer "B.Cu") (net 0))
 (segment (start 103.68 79.6) (end 103.68 76.01) (width 0.4) (layer "B.Cu") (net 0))
 (segment (start 140.49 80.725) (end 141.77 79.445) (width 0.4) (layer "B.Cu") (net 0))
 (segment (start 143.03 76.06) (end 141.77 74.8) (width 0.4) (layer "B.Cu") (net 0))
 (segment (start 132.87 80.725) (end 134.14 79.455) (width 0.4) (layer "B.Cu") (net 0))
 (segment (start 127.79 80.725) (end 127.8091 80.725) (width 0.4) (layer "B.Cu") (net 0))
 (segment (start 127.79 76.05) (end 126.52 74.78) (width 0.4) (layer "B.Cu") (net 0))
 (segment (start 146.84 79.49) (end 146.84 76.02) (width 0.4) (layer "B.Cu") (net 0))
 (segment (start 145.57 78.185) (end 145.57 76.07) (width 0.4) (layer "B.Cu") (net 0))
 (segment (start 115.09 76.05) (end 113.83 74.79) (width 0.4) (layer "B.Cu") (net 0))
 (segment (start 135.41 75.99) (end 134.16 74.74) (width 0.4) (layer "B.Cu") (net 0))
 (segment (start 120.17 70.04) (end 120.17 70.035) (width 0.4) (layer "B.Cu") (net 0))
 (segment (start 139.22 74.76) (end 139.22 71.26) (width 0.4) (layer "B.Cu") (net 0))
 (segment (start 100.94 71.485) (end 102.39 70.035) (width 0.4) (layer "B.Cu") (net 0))
 (segment (start 107.47 74.69) (end 107.47 72.575) (width 0.4) (layer "B.Cu") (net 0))
 (segment (start 132.87 78.185) (end 132.87 76) (width 0.4) (layer "B.Cu") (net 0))
 (segment (start 157.1 76.66) (end 154.76 76.66) (width 0.6) (layer "B.Cu") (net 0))
 (segment (start 146.82 71.325) (end 148.11 70.035) (width 0.4) (layer "B.Cu") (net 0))
 (segment (start 153.76 75.66) (end 153.76 74.63) (width 0.6) (layer "B.Cu") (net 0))
 (segment (start 100.94 76.735) (end 100.94 71.485) (width 0.4) (layer "B.Cu") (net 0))
 (segment (start 126.52 74.78) (end 126.52 71.305) (width 0.4) (layer "B.Cu") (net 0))
 (segment (start 143.03 74.79) (end 143.03 72.575) (width 0.4) (layer "B.Cu") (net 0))
 (segment (start 112.55 74.73) (end 112.55 72.575) (width 0.4) (layer "B.Cu") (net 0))
 (segment (start 140.49 74.79) (end 140.49 72.575) (width 0.4) (layer "B.Cu") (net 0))
 (segment (start 112.55 76.03) (end 111.28 74.76) (width 0.4) (layer "B.Cu") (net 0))
 (segment (start 129.04 79.4941) (end 129.04 76.01) (width 0.4) (layer "B.Cu") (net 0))
 (segment (start 139.22 71.26) (end 140.445 70.035) (width 0.4) (layer "B.Cu") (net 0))
 (segment (start 106.19 75.98) (end 104.93 74.72) (width 0.4) (layer "B.Cu") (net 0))
 (segment (start 103.65 74.72) (end 103.65 71.3) (width 0.4) (layer "B.Cu") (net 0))
 (segment (start 125.25 80.71) (end 126.5 79.46) (width 0.4) (layer "B.Cu") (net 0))
 (segment (start 158.09 68.99) (end 158.09 75.67) (width 0.6) (layer "B.Cu") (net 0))
 (segment (start 110.01 75.94) (end 108.76 74.69) (width 0.4) (layer "B.Cu") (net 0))
 (segment (start 113.83 74.79) (end 113.83 71.28) (width 0.4) (layer "B.Cu") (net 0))
 (segment (start 112.55 80.725) (end 112.555 80.725) (width 0.4) (layer "B.Cu") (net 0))
 (segment (start 102.555 80.725) (end 103.68 79.6) (width 0.4) (layer "B.Cu") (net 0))
 (segment (start 136.68 79.455) (end 136.68 76.03) (width 0.4) (layer "B.Cu") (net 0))
 (segment (start 102.39 74.72) (end 102.39 72.575) (width 0.4) (layer "B.Cu") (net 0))
 (segment (start 148.11 76.07) (end 146.82 74.78) (width 0.4) (layer "B.Cu") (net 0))
 (segment (start 103.68 76.01) (end 102.39 74.72) (width 0.4) (layer "B.Cu") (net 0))
 (segment (start 103.65 71.3) (end 104.59 70.36) (width 0.4) (layer "B.Cu") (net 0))
 (segment (start 123.98 71.29) (end 125.235 70.035) (width 0.4) (layer "B.Cu") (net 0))
 (segment (start 120.17 80.725) (end 121.44 79.455) (width 0.4) (layer "B.Cu") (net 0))
 (segment (start 144.3 76.06) (end 143.03 74.79) (width 0.4) (layer "B.Cu") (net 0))
 (segment (start 121.44 79.455) (end 121.44 76.02) (width 0.4) (layer "B.Cu") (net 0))
 (segment (start 112.55 78.185) (end 112.55 76.03) (width 0.4) (layer "B.Cu") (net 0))
 (segment (start 135.41 78.185) (end 135.41 75.99) (width 0.4) (layer "B.Cu") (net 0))
 (segment (start 122.71 78.185) (end 122.71 75.99) (width 0.4) (layer "B.Cu") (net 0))
 (segment (start 99.3 74.56) (end 99.3 77.63) (width 0.6) (layer "B.Cu") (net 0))
 (segment (start 144.3 74.8) (end 144.3 71.305) (width 0.4) (layer "B.Cu") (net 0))
 (segment (start 145.605 80.725) (end 146.84 79.49) (width 0.4) (layer "B.Cu") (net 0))
 (segment (start 136.7 71.285) (end 137.95 70.035) (width 0.4) (layer "B.Cu") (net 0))
 (segment (start 150.65 76.11) (end 149.39 74.85) (width 0.4) (layer "B.Cu") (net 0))
 (segment (start 149.36 76.05) (end 148.11 74.8) (width 0.4) (layer "B.Cu") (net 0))
 (segment (start 112.555 80.725) (end 113.84 79.44) (width 0.4) (layer "B.Cu") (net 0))
 (segment (start 118.91 76.05) (end 117.63 74.77) (width 0.4) (layer "B.Cu") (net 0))
 (segment (start 129.07 74.75) (end 129.07 71.295) (width 0.4) (layer "B.Cu") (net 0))
 (segment (start 139.2 79.475) (end 139.2 76.01) (width 0.4) (layer "B.Cu") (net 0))
 (segment (start 125.25 80.725) (end 125.25 80.71) (width 0.4) (layer "B.Cu") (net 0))
 (segment (start 126.5 76.06) (end 125.25 74.81) (width 0.4) (layer "B.Cu") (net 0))
 (segment (start 143.03 80.725) (end 144.3 79.455) (width 0.4) (layer "B.Cu") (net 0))
 (segment (start 141.77 79.445) (end 141.77 76.07) (width 0.4) (layer "B.Cu") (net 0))
 (segment (start 115.09 74.76) (end 115.09 72.575) (width 0.4) (layer "B.Cu") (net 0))
 (segment (start 145.57 76.07) (end 144.3 74.8) (width 0.4) (layer "B.Cu") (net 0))
 (segment (start 134.16 74.74) (end 134.16 71.285) (width 0.4) (layer "B.Cu") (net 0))
 (segment (start 115.09 80.725) (end 116.36 79.455) (width 0.4) (layer "B.Cu") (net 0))
 (segment (start 115.075 70.035) (end 115.09 70.035) (width 0.4) (layer "B.Cu") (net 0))
 (segment (start 132.87 76) (end 131.62 74.75) (width 0.4) (layer "B.Cu") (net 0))
 (segment (start 131.62 71.285) (end 132.87 70.035) (width 0.4) (layer "B.Cu") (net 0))
 (segment (start 125.25 78.185) (end 125.25 76.04) (width 0.4) (layer "B.Cu") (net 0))
 (segment (start 121.45 71.295) (end 122.71 70.035) (width 0.4) (layer "B.Cu") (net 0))
 (segment (start 125.25 76.04) (end 123.98 74.77) (width 0.4) (layer "B.Cu") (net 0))
 (segment (start 135.41 80.725) (end 136.68 79.455) (width 0.4) (layer "B.Cu") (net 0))
 (segment (start 137.95 80.725) (end 139.2 79.475) (width 0.4) (layer "B.Cu") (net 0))
 (segment (start 137.95 74.76) (end 137.95 72.575) (width 0.4) (layer "B.Cu") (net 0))
 (segment (start 113.83 71.28) (end 115.075 70.035) (width 0.4) (layer "B.Cu") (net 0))
 (segment (start 149.39 71.295) (end 150.65 70.035) (width 0.4) (layer "B.Cu") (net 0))
 (segment (start 113.84 76.02) (end 112.55 74.73) (width 0.4) (layer "B.Cu") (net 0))
 (segment (start 121.44 76.02) (end 120.17 74.75) (width 0.4) (layer "B.Cu") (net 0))
 (segment (start 148.11 74.8) (end 148.11 72.575) (width 0.4) (layer "B.Cu") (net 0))
 (segment (start 131.58 76.01) (end 130.33 74.76) (width 0.4) (layer "B.Cu") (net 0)))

